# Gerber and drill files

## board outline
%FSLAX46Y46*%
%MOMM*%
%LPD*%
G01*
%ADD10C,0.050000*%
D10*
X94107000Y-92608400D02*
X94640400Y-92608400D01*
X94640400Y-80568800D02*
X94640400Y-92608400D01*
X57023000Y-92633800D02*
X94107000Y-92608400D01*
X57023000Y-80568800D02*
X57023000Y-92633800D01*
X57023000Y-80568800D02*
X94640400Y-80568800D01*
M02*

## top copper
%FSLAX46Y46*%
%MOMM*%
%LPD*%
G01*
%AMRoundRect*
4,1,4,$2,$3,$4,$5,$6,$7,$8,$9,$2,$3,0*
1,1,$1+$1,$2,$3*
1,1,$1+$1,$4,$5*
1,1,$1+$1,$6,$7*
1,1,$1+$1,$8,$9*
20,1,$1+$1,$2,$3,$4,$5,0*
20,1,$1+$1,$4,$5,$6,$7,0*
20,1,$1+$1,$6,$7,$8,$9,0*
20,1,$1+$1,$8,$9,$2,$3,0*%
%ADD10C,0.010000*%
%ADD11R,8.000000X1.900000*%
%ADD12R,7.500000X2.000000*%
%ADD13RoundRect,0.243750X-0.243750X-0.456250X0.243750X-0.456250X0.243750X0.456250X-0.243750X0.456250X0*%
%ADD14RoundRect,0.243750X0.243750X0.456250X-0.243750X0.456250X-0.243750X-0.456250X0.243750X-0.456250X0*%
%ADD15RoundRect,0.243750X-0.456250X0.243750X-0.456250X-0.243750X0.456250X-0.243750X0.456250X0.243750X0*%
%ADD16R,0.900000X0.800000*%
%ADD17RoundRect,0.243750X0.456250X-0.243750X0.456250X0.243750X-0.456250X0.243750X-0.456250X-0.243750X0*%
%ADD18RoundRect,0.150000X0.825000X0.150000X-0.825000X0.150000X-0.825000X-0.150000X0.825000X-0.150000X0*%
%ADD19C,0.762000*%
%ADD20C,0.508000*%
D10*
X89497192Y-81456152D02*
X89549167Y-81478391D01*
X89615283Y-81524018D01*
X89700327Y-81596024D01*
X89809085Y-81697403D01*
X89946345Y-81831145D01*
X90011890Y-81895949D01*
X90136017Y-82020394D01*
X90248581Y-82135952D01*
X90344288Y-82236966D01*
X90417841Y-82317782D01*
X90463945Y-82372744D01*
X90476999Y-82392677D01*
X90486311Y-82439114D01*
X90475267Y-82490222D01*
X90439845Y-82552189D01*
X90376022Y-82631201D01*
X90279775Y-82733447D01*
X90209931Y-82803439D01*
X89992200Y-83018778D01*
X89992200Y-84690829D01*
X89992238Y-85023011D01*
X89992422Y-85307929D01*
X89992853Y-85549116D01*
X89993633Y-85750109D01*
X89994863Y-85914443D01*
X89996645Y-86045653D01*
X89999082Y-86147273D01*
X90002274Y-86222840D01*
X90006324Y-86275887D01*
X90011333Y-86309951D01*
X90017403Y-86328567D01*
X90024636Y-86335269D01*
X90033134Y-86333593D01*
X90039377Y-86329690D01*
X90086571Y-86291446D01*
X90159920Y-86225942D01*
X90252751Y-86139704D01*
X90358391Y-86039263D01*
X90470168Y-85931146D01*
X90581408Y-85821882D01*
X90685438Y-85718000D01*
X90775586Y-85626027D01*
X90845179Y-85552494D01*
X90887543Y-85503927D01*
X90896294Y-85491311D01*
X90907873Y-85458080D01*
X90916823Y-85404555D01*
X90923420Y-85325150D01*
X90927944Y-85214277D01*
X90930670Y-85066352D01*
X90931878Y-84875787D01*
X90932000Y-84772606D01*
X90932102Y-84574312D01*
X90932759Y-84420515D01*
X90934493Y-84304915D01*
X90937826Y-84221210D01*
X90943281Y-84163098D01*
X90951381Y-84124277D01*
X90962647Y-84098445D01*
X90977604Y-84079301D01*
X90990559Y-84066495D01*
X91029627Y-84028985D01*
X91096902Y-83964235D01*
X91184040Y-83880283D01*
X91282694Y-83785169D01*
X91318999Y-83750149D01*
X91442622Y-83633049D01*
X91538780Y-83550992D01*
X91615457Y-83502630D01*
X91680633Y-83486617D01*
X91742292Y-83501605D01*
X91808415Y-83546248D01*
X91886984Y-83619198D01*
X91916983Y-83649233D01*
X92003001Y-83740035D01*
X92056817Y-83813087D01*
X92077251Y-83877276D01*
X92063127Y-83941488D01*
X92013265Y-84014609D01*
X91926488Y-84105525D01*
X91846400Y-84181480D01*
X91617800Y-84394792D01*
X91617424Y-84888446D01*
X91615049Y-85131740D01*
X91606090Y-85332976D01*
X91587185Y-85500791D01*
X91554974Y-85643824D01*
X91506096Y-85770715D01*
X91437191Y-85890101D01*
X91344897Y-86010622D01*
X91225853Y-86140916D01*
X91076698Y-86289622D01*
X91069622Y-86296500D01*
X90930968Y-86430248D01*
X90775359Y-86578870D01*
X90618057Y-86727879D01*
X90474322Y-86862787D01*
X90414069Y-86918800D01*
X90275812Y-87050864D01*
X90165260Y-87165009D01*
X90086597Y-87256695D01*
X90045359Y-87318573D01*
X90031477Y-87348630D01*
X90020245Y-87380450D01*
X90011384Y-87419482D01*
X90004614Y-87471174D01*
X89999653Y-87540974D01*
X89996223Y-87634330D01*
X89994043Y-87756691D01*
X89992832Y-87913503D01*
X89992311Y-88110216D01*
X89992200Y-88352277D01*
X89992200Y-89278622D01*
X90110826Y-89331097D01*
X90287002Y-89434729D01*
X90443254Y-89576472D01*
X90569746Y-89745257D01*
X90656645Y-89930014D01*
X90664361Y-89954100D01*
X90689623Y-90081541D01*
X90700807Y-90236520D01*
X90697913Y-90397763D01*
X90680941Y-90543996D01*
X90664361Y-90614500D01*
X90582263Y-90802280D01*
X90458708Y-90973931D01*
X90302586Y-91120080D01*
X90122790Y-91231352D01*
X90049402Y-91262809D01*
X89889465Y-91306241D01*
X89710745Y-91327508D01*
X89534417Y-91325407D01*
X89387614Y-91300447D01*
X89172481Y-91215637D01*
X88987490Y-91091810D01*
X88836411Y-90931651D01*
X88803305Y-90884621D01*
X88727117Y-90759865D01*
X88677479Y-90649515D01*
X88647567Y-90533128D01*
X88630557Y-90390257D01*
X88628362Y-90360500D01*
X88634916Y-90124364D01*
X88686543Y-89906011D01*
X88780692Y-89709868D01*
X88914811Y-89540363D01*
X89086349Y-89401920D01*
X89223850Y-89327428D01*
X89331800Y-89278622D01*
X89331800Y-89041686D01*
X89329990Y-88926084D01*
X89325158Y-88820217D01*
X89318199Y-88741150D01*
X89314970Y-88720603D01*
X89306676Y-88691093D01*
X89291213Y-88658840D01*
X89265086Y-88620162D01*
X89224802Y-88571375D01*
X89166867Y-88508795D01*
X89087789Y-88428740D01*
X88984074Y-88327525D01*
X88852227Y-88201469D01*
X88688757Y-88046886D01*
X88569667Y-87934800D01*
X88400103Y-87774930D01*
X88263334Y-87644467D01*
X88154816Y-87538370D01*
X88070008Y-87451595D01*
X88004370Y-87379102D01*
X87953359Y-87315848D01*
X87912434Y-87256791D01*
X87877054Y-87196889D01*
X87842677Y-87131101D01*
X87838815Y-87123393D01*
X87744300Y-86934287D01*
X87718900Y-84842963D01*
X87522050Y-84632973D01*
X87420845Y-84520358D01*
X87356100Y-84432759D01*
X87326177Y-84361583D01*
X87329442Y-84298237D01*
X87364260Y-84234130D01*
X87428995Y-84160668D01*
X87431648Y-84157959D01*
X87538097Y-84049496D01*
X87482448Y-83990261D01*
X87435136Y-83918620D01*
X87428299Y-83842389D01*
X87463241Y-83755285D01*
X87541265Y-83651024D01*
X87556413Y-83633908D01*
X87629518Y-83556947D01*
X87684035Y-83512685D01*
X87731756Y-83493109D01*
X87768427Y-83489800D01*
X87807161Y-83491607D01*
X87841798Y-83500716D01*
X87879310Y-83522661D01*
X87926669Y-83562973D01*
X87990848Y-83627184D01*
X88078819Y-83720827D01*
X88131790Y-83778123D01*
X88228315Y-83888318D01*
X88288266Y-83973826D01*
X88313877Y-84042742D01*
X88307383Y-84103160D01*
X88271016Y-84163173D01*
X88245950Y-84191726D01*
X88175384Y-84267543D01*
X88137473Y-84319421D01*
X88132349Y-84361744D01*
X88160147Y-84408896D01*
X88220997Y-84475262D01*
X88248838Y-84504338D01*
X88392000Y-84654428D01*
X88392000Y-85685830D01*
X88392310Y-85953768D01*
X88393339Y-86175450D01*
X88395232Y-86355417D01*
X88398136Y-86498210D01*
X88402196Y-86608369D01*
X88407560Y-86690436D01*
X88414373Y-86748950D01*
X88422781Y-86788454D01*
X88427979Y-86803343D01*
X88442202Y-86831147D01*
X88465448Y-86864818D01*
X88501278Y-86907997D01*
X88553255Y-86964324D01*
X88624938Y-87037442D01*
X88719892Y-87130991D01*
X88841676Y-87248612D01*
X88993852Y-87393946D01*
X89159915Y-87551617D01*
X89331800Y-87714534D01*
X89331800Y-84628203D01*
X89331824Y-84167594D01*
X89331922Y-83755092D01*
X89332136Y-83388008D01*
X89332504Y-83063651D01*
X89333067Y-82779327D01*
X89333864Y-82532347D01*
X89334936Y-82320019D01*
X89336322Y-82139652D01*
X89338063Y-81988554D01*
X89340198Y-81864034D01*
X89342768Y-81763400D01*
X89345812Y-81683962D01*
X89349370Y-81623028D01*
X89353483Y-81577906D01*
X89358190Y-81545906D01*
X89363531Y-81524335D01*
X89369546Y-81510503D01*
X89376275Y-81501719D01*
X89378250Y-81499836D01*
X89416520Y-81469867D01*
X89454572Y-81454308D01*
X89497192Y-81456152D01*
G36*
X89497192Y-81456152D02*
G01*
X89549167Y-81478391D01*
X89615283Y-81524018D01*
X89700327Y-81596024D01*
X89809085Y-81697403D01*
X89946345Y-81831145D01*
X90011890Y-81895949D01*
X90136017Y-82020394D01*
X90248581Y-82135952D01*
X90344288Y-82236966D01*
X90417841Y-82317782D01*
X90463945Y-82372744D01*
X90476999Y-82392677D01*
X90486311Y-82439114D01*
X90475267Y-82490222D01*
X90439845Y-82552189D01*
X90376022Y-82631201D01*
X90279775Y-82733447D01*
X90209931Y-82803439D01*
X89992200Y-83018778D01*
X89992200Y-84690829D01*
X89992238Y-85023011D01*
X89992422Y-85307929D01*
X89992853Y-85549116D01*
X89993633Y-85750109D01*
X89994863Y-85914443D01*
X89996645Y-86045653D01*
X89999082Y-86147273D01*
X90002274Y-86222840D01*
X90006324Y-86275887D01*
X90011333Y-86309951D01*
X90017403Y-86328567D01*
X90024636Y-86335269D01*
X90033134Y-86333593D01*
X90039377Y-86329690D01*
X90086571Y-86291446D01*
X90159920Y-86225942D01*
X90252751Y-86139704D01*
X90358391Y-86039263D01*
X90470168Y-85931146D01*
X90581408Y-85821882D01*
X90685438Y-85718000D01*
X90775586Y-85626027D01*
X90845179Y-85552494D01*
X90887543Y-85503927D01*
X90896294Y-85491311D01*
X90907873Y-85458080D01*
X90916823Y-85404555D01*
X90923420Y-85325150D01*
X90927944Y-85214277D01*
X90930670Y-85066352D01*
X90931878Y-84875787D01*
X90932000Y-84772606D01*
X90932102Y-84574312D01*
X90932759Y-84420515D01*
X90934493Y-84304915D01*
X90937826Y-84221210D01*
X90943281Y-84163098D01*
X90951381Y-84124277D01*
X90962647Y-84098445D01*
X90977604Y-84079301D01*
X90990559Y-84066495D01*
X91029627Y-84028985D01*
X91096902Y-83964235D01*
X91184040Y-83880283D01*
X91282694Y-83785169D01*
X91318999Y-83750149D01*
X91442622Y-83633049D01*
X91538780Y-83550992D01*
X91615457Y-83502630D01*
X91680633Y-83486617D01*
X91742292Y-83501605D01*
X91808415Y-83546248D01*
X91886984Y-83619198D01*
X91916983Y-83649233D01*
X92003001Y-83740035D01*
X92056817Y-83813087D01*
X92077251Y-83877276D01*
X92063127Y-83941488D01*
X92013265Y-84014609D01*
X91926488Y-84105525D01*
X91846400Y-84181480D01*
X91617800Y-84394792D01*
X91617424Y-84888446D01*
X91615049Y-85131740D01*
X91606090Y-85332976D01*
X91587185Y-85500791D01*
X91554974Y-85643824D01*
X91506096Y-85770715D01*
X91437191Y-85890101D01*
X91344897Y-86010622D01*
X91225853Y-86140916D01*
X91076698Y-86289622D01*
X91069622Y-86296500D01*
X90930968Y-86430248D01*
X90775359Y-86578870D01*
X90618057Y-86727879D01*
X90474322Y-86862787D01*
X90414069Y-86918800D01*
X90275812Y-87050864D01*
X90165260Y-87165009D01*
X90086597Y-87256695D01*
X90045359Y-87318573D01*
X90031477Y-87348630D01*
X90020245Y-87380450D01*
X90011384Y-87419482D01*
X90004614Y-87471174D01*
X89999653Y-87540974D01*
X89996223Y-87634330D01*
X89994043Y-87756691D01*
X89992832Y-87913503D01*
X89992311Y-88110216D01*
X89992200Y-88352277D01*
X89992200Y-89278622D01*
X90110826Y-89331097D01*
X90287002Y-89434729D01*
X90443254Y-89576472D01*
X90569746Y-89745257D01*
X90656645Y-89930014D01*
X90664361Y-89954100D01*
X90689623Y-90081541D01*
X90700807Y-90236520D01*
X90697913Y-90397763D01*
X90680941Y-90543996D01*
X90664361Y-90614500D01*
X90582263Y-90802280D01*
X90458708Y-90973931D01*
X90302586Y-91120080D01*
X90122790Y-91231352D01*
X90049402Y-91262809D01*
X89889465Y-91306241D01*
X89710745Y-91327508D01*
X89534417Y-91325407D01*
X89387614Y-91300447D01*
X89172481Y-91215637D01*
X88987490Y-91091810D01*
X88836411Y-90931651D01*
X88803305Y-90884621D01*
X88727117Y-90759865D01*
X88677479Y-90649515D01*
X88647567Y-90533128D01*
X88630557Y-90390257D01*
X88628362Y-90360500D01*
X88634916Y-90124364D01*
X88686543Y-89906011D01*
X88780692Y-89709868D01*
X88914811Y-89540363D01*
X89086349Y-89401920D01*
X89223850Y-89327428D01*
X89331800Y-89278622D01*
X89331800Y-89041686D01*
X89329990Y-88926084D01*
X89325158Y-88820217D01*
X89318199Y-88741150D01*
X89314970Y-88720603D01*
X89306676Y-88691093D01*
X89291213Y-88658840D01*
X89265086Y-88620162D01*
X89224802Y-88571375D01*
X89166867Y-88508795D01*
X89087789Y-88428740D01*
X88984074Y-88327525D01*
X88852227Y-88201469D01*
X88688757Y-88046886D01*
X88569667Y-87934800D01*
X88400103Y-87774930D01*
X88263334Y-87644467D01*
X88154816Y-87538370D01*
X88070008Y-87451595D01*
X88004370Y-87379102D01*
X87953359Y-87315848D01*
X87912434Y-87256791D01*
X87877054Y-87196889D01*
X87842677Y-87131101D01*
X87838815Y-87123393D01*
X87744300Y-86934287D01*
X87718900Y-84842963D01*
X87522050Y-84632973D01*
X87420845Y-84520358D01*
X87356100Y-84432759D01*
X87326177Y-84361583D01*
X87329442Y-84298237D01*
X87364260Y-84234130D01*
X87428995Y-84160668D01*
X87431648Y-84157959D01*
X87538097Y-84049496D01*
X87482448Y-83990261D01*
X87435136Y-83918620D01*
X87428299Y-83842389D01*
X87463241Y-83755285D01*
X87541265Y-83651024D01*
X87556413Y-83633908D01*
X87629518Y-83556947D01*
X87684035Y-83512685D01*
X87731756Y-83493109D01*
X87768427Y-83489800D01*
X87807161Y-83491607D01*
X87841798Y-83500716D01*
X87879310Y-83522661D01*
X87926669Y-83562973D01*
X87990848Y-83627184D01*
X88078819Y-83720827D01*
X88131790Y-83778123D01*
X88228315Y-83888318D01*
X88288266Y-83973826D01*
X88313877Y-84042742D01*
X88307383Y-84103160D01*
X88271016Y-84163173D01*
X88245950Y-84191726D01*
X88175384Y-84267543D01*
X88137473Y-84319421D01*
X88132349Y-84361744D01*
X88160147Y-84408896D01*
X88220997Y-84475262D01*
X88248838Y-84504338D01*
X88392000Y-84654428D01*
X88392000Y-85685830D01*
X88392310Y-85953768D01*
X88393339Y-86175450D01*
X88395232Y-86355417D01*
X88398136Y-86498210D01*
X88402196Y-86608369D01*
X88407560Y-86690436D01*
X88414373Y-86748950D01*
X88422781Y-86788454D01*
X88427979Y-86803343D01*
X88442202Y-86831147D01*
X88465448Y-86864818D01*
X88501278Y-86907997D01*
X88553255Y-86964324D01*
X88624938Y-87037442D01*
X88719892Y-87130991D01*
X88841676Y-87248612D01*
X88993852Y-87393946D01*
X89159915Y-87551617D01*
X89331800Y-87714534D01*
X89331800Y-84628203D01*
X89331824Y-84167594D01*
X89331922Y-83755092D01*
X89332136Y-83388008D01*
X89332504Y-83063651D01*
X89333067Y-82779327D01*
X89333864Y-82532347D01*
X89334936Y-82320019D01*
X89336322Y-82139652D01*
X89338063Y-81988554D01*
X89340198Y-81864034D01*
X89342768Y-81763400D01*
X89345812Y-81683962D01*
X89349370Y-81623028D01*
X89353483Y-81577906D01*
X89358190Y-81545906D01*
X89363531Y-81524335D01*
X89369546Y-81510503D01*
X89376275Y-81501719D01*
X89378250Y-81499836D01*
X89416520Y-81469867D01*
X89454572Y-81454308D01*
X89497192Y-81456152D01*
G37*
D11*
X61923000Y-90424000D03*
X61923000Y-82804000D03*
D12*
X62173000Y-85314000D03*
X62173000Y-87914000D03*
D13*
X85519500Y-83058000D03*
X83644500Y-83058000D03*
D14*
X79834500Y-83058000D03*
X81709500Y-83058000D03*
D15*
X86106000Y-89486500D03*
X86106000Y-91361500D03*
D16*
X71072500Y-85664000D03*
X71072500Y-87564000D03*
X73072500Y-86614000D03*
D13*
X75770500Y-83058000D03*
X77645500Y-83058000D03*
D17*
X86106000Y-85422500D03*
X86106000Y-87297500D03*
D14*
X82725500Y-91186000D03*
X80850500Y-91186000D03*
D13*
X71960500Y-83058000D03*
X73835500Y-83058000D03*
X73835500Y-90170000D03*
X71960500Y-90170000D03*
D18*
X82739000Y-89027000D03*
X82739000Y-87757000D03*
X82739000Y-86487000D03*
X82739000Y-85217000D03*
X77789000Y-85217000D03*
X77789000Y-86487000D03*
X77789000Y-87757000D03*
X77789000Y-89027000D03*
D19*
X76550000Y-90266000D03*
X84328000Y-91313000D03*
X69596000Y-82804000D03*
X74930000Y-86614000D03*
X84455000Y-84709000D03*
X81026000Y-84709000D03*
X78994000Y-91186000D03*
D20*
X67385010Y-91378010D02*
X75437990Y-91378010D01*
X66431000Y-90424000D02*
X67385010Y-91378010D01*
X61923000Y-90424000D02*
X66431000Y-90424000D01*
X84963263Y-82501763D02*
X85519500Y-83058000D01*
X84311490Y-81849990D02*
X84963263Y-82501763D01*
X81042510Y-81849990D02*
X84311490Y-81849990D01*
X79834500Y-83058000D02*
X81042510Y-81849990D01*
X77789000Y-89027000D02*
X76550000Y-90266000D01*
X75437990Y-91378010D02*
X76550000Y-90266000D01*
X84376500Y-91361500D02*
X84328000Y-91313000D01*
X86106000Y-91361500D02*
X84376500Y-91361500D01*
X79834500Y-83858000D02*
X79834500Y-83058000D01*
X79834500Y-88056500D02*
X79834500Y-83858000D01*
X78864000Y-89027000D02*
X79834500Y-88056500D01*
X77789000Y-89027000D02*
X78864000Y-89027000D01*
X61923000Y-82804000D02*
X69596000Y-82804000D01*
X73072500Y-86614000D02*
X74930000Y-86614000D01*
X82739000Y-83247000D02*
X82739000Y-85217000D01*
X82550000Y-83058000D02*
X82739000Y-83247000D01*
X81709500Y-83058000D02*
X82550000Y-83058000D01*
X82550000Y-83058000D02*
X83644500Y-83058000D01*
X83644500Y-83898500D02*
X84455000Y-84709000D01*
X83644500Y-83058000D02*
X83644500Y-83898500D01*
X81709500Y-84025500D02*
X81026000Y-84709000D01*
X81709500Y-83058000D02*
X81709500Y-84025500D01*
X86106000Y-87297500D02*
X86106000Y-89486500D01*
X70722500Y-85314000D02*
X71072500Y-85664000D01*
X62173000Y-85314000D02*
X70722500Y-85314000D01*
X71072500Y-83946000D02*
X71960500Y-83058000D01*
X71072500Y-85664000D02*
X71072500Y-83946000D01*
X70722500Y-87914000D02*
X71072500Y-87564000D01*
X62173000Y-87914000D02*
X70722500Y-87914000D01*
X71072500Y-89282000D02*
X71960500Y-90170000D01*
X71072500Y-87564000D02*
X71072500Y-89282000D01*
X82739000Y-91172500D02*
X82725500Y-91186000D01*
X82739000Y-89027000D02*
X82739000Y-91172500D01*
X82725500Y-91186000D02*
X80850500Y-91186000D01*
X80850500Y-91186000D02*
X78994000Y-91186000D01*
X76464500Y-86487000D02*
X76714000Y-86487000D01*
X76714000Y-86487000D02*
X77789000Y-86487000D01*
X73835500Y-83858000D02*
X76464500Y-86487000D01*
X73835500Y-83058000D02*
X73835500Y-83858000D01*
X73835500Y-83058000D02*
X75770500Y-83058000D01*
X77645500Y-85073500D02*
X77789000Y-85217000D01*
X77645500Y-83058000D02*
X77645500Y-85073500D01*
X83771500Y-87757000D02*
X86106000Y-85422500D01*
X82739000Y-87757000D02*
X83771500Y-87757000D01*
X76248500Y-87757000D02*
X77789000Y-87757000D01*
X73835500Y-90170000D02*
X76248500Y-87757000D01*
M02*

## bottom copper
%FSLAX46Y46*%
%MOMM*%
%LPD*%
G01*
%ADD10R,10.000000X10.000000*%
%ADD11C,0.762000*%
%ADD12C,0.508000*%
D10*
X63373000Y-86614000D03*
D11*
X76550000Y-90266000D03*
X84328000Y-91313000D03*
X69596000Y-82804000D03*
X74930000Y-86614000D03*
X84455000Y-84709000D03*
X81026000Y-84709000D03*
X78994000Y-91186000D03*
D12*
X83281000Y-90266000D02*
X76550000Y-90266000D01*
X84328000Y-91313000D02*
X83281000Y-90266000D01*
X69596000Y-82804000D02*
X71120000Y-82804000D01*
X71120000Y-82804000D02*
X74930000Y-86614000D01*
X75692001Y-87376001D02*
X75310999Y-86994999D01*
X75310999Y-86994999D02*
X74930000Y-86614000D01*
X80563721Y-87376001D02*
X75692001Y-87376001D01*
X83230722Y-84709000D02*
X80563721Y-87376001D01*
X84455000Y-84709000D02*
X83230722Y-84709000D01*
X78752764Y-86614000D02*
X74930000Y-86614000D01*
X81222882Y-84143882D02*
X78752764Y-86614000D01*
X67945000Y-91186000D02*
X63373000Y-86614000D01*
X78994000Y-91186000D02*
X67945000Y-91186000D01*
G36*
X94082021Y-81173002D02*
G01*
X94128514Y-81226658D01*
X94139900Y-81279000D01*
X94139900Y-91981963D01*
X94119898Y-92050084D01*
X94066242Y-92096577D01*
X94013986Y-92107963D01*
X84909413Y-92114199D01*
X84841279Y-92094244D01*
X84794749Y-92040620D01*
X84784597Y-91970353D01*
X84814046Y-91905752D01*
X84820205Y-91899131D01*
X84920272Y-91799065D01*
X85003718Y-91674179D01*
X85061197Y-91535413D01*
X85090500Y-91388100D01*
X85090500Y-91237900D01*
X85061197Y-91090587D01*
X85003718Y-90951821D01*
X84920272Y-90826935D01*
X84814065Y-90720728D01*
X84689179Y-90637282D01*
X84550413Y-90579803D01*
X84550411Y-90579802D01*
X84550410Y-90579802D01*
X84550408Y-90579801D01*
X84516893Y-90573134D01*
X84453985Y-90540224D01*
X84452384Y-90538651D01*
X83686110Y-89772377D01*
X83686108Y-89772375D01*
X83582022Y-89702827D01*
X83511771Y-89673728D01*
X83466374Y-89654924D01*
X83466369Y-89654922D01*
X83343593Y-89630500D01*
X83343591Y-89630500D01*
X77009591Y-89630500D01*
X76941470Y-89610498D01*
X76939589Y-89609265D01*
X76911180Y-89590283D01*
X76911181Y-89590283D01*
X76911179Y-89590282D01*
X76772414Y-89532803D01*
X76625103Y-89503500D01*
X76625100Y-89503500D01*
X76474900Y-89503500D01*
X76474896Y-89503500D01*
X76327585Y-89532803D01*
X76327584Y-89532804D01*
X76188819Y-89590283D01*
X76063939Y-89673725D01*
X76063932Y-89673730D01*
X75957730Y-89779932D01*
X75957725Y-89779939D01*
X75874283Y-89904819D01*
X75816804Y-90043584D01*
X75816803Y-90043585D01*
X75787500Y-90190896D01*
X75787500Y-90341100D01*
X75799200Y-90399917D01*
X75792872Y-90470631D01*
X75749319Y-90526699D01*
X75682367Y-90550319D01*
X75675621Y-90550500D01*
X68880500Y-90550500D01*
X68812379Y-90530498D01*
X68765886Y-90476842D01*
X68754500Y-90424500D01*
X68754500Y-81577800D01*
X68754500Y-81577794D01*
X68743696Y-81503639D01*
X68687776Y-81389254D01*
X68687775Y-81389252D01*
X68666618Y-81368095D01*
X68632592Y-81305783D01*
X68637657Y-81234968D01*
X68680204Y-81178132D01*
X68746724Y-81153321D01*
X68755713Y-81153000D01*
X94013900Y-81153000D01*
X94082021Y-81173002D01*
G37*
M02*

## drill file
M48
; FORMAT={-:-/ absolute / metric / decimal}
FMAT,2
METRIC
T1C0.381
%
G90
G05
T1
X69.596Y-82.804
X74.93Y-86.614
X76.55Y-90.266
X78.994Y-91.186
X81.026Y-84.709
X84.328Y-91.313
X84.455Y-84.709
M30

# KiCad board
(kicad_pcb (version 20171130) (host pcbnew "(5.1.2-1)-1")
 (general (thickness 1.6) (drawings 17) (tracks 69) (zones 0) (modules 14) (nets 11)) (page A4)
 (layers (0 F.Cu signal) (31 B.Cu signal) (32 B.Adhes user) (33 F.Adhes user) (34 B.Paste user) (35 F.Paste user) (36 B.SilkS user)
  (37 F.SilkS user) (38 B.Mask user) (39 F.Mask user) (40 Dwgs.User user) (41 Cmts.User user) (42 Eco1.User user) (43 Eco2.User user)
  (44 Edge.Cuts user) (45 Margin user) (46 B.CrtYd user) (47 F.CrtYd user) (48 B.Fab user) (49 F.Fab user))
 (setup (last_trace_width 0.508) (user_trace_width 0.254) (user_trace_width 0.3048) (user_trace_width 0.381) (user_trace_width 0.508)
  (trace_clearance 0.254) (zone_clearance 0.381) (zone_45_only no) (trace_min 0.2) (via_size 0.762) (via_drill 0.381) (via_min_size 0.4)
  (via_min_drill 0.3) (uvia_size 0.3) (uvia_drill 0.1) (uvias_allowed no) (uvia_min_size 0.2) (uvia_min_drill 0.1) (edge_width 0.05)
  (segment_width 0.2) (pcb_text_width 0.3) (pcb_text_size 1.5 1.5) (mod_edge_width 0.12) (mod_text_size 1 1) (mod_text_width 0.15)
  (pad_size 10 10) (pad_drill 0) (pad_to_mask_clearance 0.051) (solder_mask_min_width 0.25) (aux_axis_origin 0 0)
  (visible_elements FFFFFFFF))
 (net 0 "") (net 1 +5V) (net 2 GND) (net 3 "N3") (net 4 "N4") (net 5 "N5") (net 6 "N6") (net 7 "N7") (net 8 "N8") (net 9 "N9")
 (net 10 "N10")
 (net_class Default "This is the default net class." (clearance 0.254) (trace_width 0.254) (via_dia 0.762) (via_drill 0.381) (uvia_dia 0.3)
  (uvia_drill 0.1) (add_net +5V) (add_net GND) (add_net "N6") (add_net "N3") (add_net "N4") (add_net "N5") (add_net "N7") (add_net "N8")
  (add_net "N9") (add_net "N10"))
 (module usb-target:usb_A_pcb (layer F.Cu) (at 57.023 86.614 270)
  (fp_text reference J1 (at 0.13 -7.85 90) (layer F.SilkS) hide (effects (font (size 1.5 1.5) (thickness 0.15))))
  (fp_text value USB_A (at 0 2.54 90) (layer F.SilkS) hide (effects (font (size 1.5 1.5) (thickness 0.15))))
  (pad 1 connect rect (at 3.81 -4.9 270) (size 1.9 8) (layers F.Cu F.Mask) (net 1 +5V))
  (pad 4 connect rect (at -3.81 -4.9 270) (size 1.9 8) (layers F.Cu F.Mask) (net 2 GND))
  (pad 3 connect rect (at -1.3 -5.15 270) (size 2 7.5) (layers F.Cu F.Mask) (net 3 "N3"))
  (pad 2 connect rect (at 1.3 -5.15 270) (size 2 7.5) (layers F.Cu F.Mask) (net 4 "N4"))
  (pad 5 smd rect (at 0 -6.35 270) (size 10 10) (layers B.Cu B.Mask) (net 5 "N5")))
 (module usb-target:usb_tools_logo (layer F.Cu) (at 89.662 86.36)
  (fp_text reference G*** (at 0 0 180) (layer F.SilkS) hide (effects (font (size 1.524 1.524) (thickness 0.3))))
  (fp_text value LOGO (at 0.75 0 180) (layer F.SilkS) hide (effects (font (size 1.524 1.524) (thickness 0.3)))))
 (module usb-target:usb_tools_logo (layer F.Cu) (at 89.662 86.36)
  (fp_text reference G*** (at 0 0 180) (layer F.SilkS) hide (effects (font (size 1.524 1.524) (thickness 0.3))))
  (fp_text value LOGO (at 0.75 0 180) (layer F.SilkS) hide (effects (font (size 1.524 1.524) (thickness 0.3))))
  (fp_poly
   (pts (xy -0.164808 -4.903848) (xy -0.112833 -4.881609) (xy -0.046717 -4.835982) (xy 0.038327 -4.763976) (xy 0.147085 -4.662597)
    (xy 0.284345 -4.528855) (xy 0.34989 -4.464051) (xy 0.474017 -4.339606) (xy 0.586581 -4.224048) (xy 0.682288 -4.123034)
    (xy 0.755841 -4.042218) (xy 0.801945 -3.987256) (xy 0.814999 -3.967323) (xy 0.824311 -3.920886) (xy 0.813267 -3.869778)
    (xy 0.777845 -3.807811) (xy 0.714022 -3.728799) (xy 0.617775 -3.626553) (xy 0.547931 -3.556561) (xy 0.3302 -3.341222)
    (xy 0.3302 -1.669171) (xy 0.330238 -1.336989) (xy 0.330422 -1.052071) (xy 0.330853 -0.810884) (xy 0.331633 -0.609891)
    (xy 0.332863 -0.445557) (xy 0.334645 -0.314347) (xy 0.337082 -0.212727) (xy 0.340274 -0.13716) (xy 0.344324 -0.084113)
    (xy 0.349333 -0.050049) (xy 0.355403 -0.031433) (xy 0.362636 -0.024731) (xy 0.371134 -0.026407) (xy 0.377377 -0.03031)
    (xy 0.424571 -0.068554) (xy 0.49792 -0.134058) (xy 0.590751 -0.220296) (xy 0.696391 -0.320737) (xy 0.808168 -0.428854)
    (xy 0.919408 -0.538118) (xy 1.023438 -0.642) (xy 1.113586 -0.733973) (xy 1.183179 -0.807506) (xy 1.225543 -0.856073)
    (xy 1.234294 -0.868689) (xy 1.245873 -0.90192) (xy 1.254823 -0.955445) (xy 1.26142 -1.03485) (xy 1.265944 -1.145723)
    (xy 1.26867 -1.293648) (xy 1.269878 -1.484213) (xy 1.27 -1.587394) (xy 1.270102 -1.785688) (xy 1.270759 -1.939485)
    (xy 1.272493 -2.055085) (xy 1.275826 -2.13879) (xy 1.281281 -2.196902) (xy 1.289381 -2.235723) (xy 1.300647 -2.261555)
    (xy 1.315604 -2.280699) (xy 1.328559 -2.293505) (xy 1.367627 -2.331015) (xy 1.434902 -2.395765) (xy 1.52204 -2.479717)
    (xy 1.620694 -2.574831) (xy 1.656999 -2.609851) (xy 1.780622 -2.726951) (xy 1.87678 -2.809008) (xy 1.953457 -2.85737)
    (xy 2.018633 -2.873383) (xy 2.080292 -2.858395) (xy 2.146415 -2.813752) (xy 2.224984 -2.740802) (xy 2.254983 -2.710767)
    (xy 2.341001 -2.619965) (xy 2.394817 -2.546913) (xy 2.415251 -2.482724) (xy 2.401127 -2.418512) (xy 2.351265 -2.345391)
    (xy 2.264488 -2.254475) (xy 2.1844 -2.17852) (xy 1.9558 -1.965208) (xy 1.955424 -1.471554) (xy 1.953049 -1.22826) (xy 1.94409 -1.027024)
    (xy 1.925185 -0.859209) (xy 1.892974 -0.716176) (xy 1.844096 -0.589285) (xy 1.775191 -0.469899) (xy 1.682897 -0.349378)
    (xy 1.563853 -0.219084) (xy 1.414698 -0.070378) (xy 1.407622 -0.0635) (xy 1.268968 0.070248) (xy 1.113359 0.21887)
    (xy 0.956057 0.367879) (xy 0.812322 0.502787) (xy 0.752069 0.5588) (xy 0.613812 0.690864) (xy 0.50326 0.805009) (xy 0.424597 0.896695)
    (xy 0.383359 0.958573) (xy 0.369477 0.98863) (xy 0.358245 1.02045) (xy 0.349384 1.059482) (xy 0.342614 1.111174) (xy 0.337653 1.180974)
    (xy 0.334223 1.27433) (xy 0.332043 1.396691) (xy 0.330832 1.553503) (xy 0.330311 1.750216) (xy 0.3302 1.992277) (xy 0.3302 2.918622)
    (xy 0.448826 2.971097) (xy 0.625002 3.074729) (xy 0.781254 3.216472) (xy 0.907746 3.385257) (xy 0.994645 3.570014) (xy 1.002361 3.5941)
    (xy 1.027623 3.721541) (xy 1.038807 3.87652) (xy 1.035913 4.037763) (xy 1.018941 4.183996) (xy 1.002361 4.2545) (xy 0.920263 4.44228)
    (xy 0.796708 4.613931) (xy 0.640586 4.76008) (xy 0.46079 4.871352) (xy 0.387402 4.902809) (xy 0.227465 4.946241) (xy 0.048745 4.967508)
    (xy -0.127583 4.965407) (xy -0.274386 4.940447) (xy -0.489519 4.855637) (xy -0.67451 4.73181) (xy -0.825589 4.571651)
    (xy -0.858695 4.524621) (xy -0.934883 4.399865) (xy -0.984521 4.289515) (xy -1.014433 4.173128) (xy -1.031443 4.030257)
    (xy -1.033638 4.0005) (xy -1.027084 3.764364) (xy -0.975457 3.546011) (xy -0.881308 3.349868) (xy -0.747189 3.180363)
    (xy -0.575651 3.04192) (xy -0.43815 2.967428) (xy -0.3302 2.918622) (xy -0.3302 2.681686) (xy -0.33201 2.566084) (xy -0.336842 2.460217)
    (xy -0.343801 2.38115) (xy -0.34703 2.360603) (xy -0.355324 2.331093) (xy -0.370787 2.29884) (xy -0.396914 2.260162)
    (xy -0.437198 2.211375) (xy -0.495133 2.148795) (xy -0.574211 2.06874) (xy -0.677926 1.967525) (xy -0.809773 1.841469)
    (xy -0.973243 1.686886) (xy -1.092333 1.5748) (xy -1.261897 1.41493) (xy -1.398666 1.284467) (xy -1.507184 1.17837)
    (xy -1.591992 1.091595) (xy -1.65763 1.019102) (xy -1.708641 0.955848) (xy -1.749566 0.896791) (xy -1.784946 0.836889)
    (xy -1.819323 0.771101) (xy -1.823185 0.763393) (xy -1.9177 0.574287) (xy -1.9431 -1.517037) (xy -2.13995 -1.727027)
    (xy -2.241155 -1.839642) (xy -2.3059 -1.927241) (xy -2.335823 -1.998417) (xy -2.332558 -2.061763) (xy -2.29774 -2.12587)
    (xy -2.233005 -2.199332) (xy -2.230352 -2.202041) (xy -2.123903 -2.310504) (xy -2.179552 -2.369739) (xy -2.226864 -2.44138)
    (xy -2.233701 -2.517611) (xy -2.198759 -2.604715) (xy -2.120735 -2.708976) (xy -2.105587 -2.726092) (xy -2.032482 -2.803053)
    (xy -1.977965 -2.847315) (xy -1.930244 -2.866891) (xy -1.893573 -2.8702) (xy -1.854839 -2.868393) (xy -1.820202 -2.859284)
    (xy -1.78269 -2.837339) (xy -1.735331 -2.797027) (xy -1.671152 -2.732816) (xy -1.583181 -2.639173) (xy -1.53021 -2.581877)
    (xy -1.433685 -2.471682) (xy -1.373734 -2.386174) (xy -1.348123 -2.317258) (xy -1.354617 -2.25684) (xy -1.390984 -2.196827)
    (xy -1.41605 -2.168274) (xy -1.486616 -2.092457) (xy -1.524527 -2.040579) (xy -1.529651 -1.998256) (xy -1.501853 -1.951104)
    (xy -1.441003 -1.884738) (xy -1.413162 -1.855662) (xy -1.27 -1.705572) (xy -1.27 -0.67417) (xy -1.26969 -0.406232)
    (xy -1.268661 -0.18455) (xy -1.266768 -0.004583) (xy -1.263864 0.13821) (xy -1.259804 0.248369) (xy -1.25444 0.330436)
    (xy -1.247627 0.38895) (xy -1.239219 0.428454) (xy -1.234021 0.443343) (xy -1.219798 0.471147) (xy -1.196552 0.504818)
    (xy -1.160722 0.547997) (xy -1.108745 0.604324) (xy -1.037062 0.677442) (xy -0.942108 0.770991) (xy -0.820324 0.888612)
    (xy -0.668148 1.033946) (xy -0.502085 1.191617) (xy -0.3302 1.354534) (xy -0.3302 -1.731797) (xy -0.330176 -2.192406)
    (xy -0.330078 -2.604908) (xy -0.329864 -2.971992) (xy -0.329496 -3.296349) (xy -0.328933 -3.580673) (xy -0.328136 -3.827653)
    (xy -0.327064 -4.039981) (xy -0.325678 -4.220348) (xy -0.323937 -4.371446) (xy -0.321802 -4.495966) (xy -0.319232 -4.5966)
    (xy -0.316188 -4.676038) (xy -0.31263 -4.736972) (xy -0.308517 -4.782094) (xy -0.30381 -4.814094) (xy -0.298469 -4.835665)
    (xy -0.292454 -4.849497) (xy -0.285725 -4.858281) (xy -0.28375 -4.860164) (xy -0.24548 -4.890133) (xy -0.207428 -4.905692)
    (xy -0.164808 -4.903848))
   (layer F.Cu) (width 0.01)))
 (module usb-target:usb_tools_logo (layer B.Cu) (at 91.567 86.487 180)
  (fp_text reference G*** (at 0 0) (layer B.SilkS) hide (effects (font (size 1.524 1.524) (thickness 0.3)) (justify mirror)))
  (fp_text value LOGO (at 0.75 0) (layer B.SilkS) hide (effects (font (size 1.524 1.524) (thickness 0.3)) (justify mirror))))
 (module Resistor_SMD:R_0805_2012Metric (layer F.Cu) (at 84.582 83.058)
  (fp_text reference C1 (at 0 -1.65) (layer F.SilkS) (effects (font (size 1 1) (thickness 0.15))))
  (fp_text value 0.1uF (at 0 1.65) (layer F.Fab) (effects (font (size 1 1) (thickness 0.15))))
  (pad 2 smd roundrect (at 0.9375 0) (size 0.975 1.4) (layers F.Cu F.Paste F.Mask) (roundrect_rratio 0.25) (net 1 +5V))
  (pad 1 smd roundrect (at -0.9375 0) (size 0.975 1.4) (layers F.Cu F.Paste F.Mask) (roundrect_rratio 0.25) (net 2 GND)))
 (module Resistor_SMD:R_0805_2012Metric (layer F.Cu) (at 80.772 83.058 180)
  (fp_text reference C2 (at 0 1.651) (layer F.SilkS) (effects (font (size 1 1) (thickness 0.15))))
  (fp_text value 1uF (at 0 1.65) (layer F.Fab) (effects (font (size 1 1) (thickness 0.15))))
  (pad 2 smd roundrect (at 0.9375 0 180) (size 0.975 1.4) (layers F.Cu F.Paste F.Mask) (roundrect_rratio 0.25) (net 1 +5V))
  (pad 1 smd roundrect (at -0.9375 0 180) (size 0.975 1.4) (layers F.Cu F.Paste F.Mask) (roundrect_rratio 0.25) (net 2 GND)))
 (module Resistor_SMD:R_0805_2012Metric (layer F.Cu) (at 86.106 90.424 270)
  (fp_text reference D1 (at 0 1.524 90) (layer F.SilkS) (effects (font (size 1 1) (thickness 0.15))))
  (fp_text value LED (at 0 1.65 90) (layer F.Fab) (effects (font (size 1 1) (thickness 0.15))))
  (pad 1 smd roundrect (at -0.9375 0 270) (size 0.975 1.4) (layers F.Cu F.Paste F.Mask) (roundrect_rratio 0.25) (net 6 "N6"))
  (pad 2 smd roundrect (at 0.9375 0 270) (size 0.975 1.4) (layers F.Cu F.Paste F.Mask) (roundrect_rratio 0.25) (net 1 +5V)))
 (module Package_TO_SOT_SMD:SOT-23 (layer F.Cu) (at 72.0725 86.614)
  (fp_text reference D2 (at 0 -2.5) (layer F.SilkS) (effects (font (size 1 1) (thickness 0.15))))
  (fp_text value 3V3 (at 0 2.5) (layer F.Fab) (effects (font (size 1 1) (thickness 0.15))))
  (pad 1 smd rect (at -1 -0.95) (size 0.9 0.8) (layers F.Cu F.Paste F.Mask) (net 3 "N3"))
  (pad 2 smd rect (at -1 0.95) (size 0.9 0.8) (layers F.Cu F.Paste F.Mask) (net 4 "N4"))
  (pad 3 smd rect (at 1 0) (size 0.9 0.8) (layers F.Cu F.Paste F.Mask) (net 2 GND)))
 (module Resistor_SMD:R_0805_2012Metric (layer F.Cu) (at 76.708 83.058)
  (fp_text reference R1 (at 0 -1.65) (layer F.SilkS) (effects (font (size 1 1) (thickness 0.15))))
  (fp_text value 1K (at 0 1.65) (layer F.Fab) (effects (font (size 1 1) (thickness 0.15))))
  (pad 1 smd roundrect (at -0.9375 0) (size 0.975 1.4) (layers F.Cu F.Paste F.Mask) (roundrect_rratio 0.25) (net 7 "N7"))
  (pad 2 smd roundrect (at 0.9375 0) (size 0.975 1.4) (layers F.Cu F.Paste F.Mask) (roundrect_rratio 0.25) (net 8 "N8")))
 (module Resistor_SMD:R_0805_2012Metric (layer F.Cu) (at 86.106 86.36 90)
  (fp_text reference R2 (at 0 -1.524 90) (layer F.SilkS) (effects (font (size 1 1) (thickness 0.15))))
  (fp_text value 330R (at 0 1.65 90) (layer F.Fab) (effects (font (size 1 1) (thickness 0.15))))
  (pad 2 smd roundrect (at 0.9375 0 90) (size 0.975 1.4) (layers F.Cu F.Paste F.Mask) (roundrect_rratio 0.25) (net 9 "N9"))
  (pad 1 smd roundrect (at -0.9375 0 90) (size 0.975 1.4) (layers F.Cu F.Paste F.Mask) (roundrect_rratio 0.25) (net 6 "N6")))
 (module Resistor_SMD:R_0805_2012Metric (layer F.Cu) (at 81.788 91.186 180)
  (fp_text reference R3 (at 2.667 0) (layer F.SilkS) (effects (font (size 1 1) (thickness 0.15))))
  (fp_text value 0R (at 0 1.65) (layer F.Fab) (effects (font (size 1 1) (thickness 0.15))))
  (pad 1 smd roundrect (at -0.9375 0 180) (size 0.975 1.4) (layers F.Cu F.Paste F.Mask) (roundrect_rratio 0.25) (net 5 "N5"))
  (pad 2 smd roundrect (at 0.9375 0 180) (size 0.975 1.4) (layers F.Cu F.Paste F.Mask) (roundrect_rratio 0.25) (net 5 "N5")))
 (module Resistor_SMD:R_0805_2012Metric (layer F.Cu) (at 72.898 83.058)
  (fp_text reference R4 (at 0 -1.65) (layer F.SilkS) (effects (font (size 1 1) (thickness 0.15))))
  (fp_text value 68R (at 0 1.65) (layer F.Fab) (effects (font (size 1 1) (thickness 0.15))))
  (pad 1 smd roundrect (at -0.9375 0) (size 0.975 1.4) (layers F.Cu F.Paste F.Mask) (roundrect_rratio 0.25) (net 3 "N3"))
  (pad 2 smd roundrect (at 0.9375 0) (size 0.975 1.4) (layers F.Cu F.Paste F.Mask) (roundrect_rratio 0.25) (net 7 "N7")))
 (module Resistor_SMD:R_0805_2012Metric (layer F.Cu) (at 72.898 90.17)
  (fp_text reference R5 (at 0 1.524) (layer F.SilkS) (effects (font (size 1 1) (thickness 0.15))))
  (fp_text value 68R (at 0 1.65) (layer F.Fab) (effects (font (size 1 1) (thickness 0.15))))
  (pad 2 smd roundrect (at 0.9375 0) (size 0.975 1.4) (layers F.Cu F.Paste F.Mask) (roundrect_rratio 0.25) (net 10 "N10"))
  (pad 1 smd roundrect (at -0.9375 0) (size 0.975 1.4) (layers F.Cu F.Paste F.Mask) (roundrect_rratio 0.25) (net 4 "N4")))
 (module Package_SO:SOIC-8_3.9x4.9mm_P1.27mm (layer F.Cu) (at 80.264 87.122 180)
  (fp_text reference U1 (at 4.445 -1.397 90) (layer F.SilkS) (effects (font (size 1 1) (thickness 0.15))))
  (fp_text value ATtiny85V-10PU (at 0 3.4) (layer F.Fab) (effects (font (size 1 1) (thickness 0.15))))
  (pad 1 smd roundrect (at -2.475 -1.905 180) (size 1.95 0.6) (layers F.Cu F.Paste F.Mask) (roundrect_rratio 0.25) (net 5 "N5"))
  (pad 2 smd roundrect (at -2.475 -0.635 180) (size 1.95 0.6) (layers F.Cu F.Paste F.Mask) (roundrect_rratio 0.25) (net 9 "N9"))
  (pad 3 smd roundrect (at -2.475 0.635 180) (size 1.95 0.6) (layers F.Cu F.Paste F.Mask) (roundrect_rratio 0.25))
  (pad 4 smd roundrect (at -2.475 1.905 180) (size 1.95 0.6) (layers F.Cu F.Paste F.Mask) (roundrect_rratio 0.25) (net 2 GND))
  (pad 5 smd roundrect (at 2.475 1.905 180) (size 1.95 0.6) (layers F.Cu F.Paste F.Mask) (roundrect_rratio 0.25) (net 8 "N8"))
  (pad 6 smd roundrect (at 2.475 0.635 180) (size 1.95 0.6) (layers F.Cu F.Paste F.Mask) (roundrect_rratio 0.25) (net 7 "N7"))
  (pad 7 smd roundrect (at 2.475 -0.635 180) (size 1.95 0.6) (layers F.Cu F.Paste F.Mask) (roundrect_rratio 0.25) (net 10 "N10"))
  (pad 8 smd roundrect (at 2.475 -1.905 180) (size 1.95 0.6) (layers F.Cu F.Paste F.Mask) (roundrect_rratio 0.25) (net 1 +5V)))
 (gr_line (start 94.107 92.6084) (end 94.6404 92.6084) (layer Edge.Cuts) (width 0.05))
 (gr_line (start 94.6404 80.5688) (end 94.6404 92.6084) (layer Edge.Cuts) (width 0.05))
 (gr_line (start 57.023 92.6338) (end 94.107 92.6084) (layer Edge.Cuts) (width 0.05))
 (gr_line (start 57.023 80.5688) (end 57.023 92.6338) (layer Edge.Cuts) (width 0.05))
 (gr_line (start 57.023 80.5688) (end 94.6404 80.5688) (layer Edge.Cuts) (width 0.05))
 (segment (start 67.38501 91.37801) (end 75.43799 91.37801) (width 0.508) (layer F.Cu) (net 1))
 (segment (start 66.431 90.424) (end 67.38501 91.37801) (width 0.508) (layer F.Cu) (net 1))
 (segment (start 61.923 90.424) (end 66.431 90.424) (width 0.508) (layer F.Cu) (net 1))
 (segment (start 84.963263 82.501763) (end 85.5195 83.058) (width 0.508) (layer F.Cu) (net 1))
 (segment (start 84.31149 81.84999) (end 84.963263 82.501763) (width 0.508) (layer F.Cu) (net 1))
 (segment (start 81.04251 81.84999) (end 84.31149 81.84999) (width 0.508) (layer F.Cu) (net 1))
 (segment (start 79.8345 83.058) (end 81.04251 81.84999) (width 0.508) (layer F.Cu) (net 1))
 (via (at 76.55 90.266) (size 0.762) (drill 0.381) (layers F.Cu B.Cu) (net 1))
 (segment (start 77.789 89.027) (end 76.55 90.266) (width 0.508) (layer F.Cu) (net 1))
 (segment (start 75.43799 91.37801) (end 76.55 90.266) (width 0.508) (layer F.Cu) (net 1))
 (via (at 84.328 91.313) (size 0.762) (drill 0.381) (layers F.Cu B.Cu) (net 1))
 (segment (start 84.3765 91.3615) (end 84.328 91.313) (width 0.508) (layer F.Cu) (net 1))
 (segment (start 86.106 91.3615) (end 84.3765 91.3615) (width 0.508) (layer F.Cu) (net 1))
 (segment (start 83.281 90.266) (end 76.55 90.266) (width 0.508) (layer B.Cu) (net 1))
 (segment (start 84.328 91.313) (end 83.281 90.266) (width 0.508) (layer B.Cu) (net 1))
 (segment (start 79.8345 83.858) (end 79.8345 83.058) (width 0.508) (layer F.Cu) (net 1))
 (segment (start 79.8345 88.0565) (end 79.8345 83.858) (width 0.508) (layer F.Cu) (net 1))
 (segment (start 78.864 89.027) (end 79.8345 88.0565) (width 0.508) (layer F.Cu) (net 1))
 (segment (start 77.789 89.027) (end 78.864 89.027) (width 0.508) (layer F.Cu) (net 1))
 (via (at 69.596 82.804) (size 0.762) (drill 0.381) (layers F.Cu B.Cu) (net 2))
 (segment (start 61.923 82.804) (end 69.596 82.804) (width 0.508) (layer F.Cu) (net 2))
 (segment (start 69.596 82.804) (end 71.12 82.804) (width 0.508) (layer B.Cu) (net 2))
 (segment (start 71.12 82.804) (end 74.93 86.614) (width 0.508) (layer B.Cu) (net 2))
 (via (at 74.93 86.614) (size 0.762) (drill 0.381) (layers F.Cu B.Cu) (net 2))
 (segment (start 73.0725 86.614) (end 74.93 86.614) (width 0.508) (layer F.Cu) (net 2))
 (segment (start 82.739 83.247) (end 82.739 85.217) (width 0.508) (layer F.Cu) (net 2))
 (segment (start 82.55 83.058) (end 82.739 83.247) (width 0.508) (layer F.Cu) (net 2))
 (segment (start 81.7095 83.058) (end 82.55 83.058) (width 0.508) (layer F.Cu) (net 2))
 (segment (start 82.55 83.058) (end 83.6445 83.058) (width 0.508) (layer F.Cu) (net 2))
 (via (at 84.455 84.709) (size 0.762) (drill 0.381) (layers F.Cu B.Cu) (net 2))
 (segment (start 83.6445 83.8985) (end 84.455 84.709) (width 0.508) (layer F.Cu) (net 2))
 (segment (start 83.6445 83.058) (end 83.6445 83.8985) (width 0.508) (layer F.Cu) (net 2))
 (segment (start 75.692001 87.376001) (end 75.310999 86.994999) (width 0.508) (layer B.Cu) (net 2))
 (segment (start 75.310999 86.994999) (end 74.93 86.614) (width 0.508) (layer B.Cu) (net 2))
 (segment (start 80.563721 87.376001) (end 75.692001 87.376001) (width 0.508) (layer B.Cu) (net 2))
 (segment (start 83.230722 84.709) (end 80.563721 87.376001) (width 0.508) (layer B.Cu) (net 2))
 (segment (start 84.455 84.709) (end 83.230722 84.709) (width 0.508) (layer B.Cu) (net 2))
 (segment (start 78.752764 86.614) (end 74.93 86.614) (width 0.508) (layer B.Cu) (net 2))
 (segment (start 81.222882 84.143882) (end 78.752764 86.614) (width 0.508) (layer B.Cu) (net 2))
 (segment (start 81.7095 84.0255) (end 81.026 84.709) (width 0.508) (layer F.Cu) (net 2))
 (via (at 81.026 84.709) (size 0.762) (drill 0.381) (layers F.Cu B.Cu) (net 2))
 (segment (start 81.7095 83.058) (end 81.7095 84.0255) (width 0.508) (layer F.Cu) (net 2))
 (segment (start 86.106 87.2975) (end 86.106 89.4865) (width 0.508) (layer F.Cu) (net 6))
 (segment (start 70.7225 85.314) (end 71.0725 85.664) (width 0.508) (layer F.Cu) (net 3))
 (segment (start 62.173 85.314) (end 70.7225 85.314) (width 0.508) (layer F.Cu) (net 3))
 (segment (start 71.0725 83.946) (end 71.9605 83.058) (width 0.508) (layer F.Cu) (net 3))
 (segment (start 71.0725 85.664) (end 71.0725 83.946) (width 0.508) (layer F.Cu) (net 3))
 (segment (start 70.7225 87.914) (end 71.0725 87.564) (width 0.508) (layer F.Cu) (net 4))
 (segment (start 62.173 87.914) (end 70.7225 87.914) (width 0.508) (layer F.Cu) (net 4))
 (segment (start 71.0725 89.282) (end 71.9605 90.17) (width 0.508) (layer F.Cu) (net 4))
 (segment (start 71.0725 87.564) (end 71.0725 89.282) (width 0.508) (layer F.Cu) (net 4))
 (segment (start 82.739 91.1725) (end 82.7255 91.186) (width 0.508) (layer F.Cu) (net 5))
 (segment (start 82.739 89.027) (end 82.739 91.1725) (width 0.508) (layer F.Cu) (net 5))
 (segment (start 82.7255 91.186) (end 80.8505 91.186) (width 0.508) (layer F.Cu) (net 5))
 (via (at 78.994 91.186) (size 0.762) (drill 0.381) (layers F.Cu B.Cu) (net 5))
 (segment (start 80.8505 91.186) (end 78.994 91.186) (width 0.508) (layer F.Cu) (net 5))
 (segment (start 67.945 91.186) (end 63.373 86.614) (width 0.508) (layer B.Cu) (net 5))
 (segment (start 78.994 91.186) (end 67.945 91.186) (width 0.508) (layer B.Cu) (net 5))
 (segment (start 76.4645 86.487) (end 76.714 86.487) (width 0.508) (layer F.Cu) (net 7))
 (segment (start 76.714 86.487) (end 77.789 86.487) (width 0.508) (layer F.Cu) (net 7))
 (segment (start 73.8355 83.858) (end 76.4645 86.487) (width 0.508) (layer F.Cu) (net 7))
 (segment (start 73.8355 83.058) (end 73.8355 83.858) (width 0.508) (layer F.Cu) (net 7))
 (segment (start 73.8355 83.058) (end 75.7705 83.058) (width 0.508) (layer F.Cu) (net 7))
 (segment (start 77.6455 85.0735) (end 77.789 85.217) (width 0.508) (layer F.Cu) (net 8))
 (segment (start 77.6455 83.058) (end 77.6455 85.0735) (width 0.508) (layer F.Cu) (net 8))
 (segment (start 83.7715 87.757) (end 86.106 85.4225) (width 0.508) (layer F.Cu) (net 9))
 (segment (start 82.739 87.757) (end 83.7715 87.757) (width 0.508) (layer F.Cu) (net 9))
 (segment (start 76.2485 87.757) (end 77.789 87.757) (width 0.508) (layer F.Cu) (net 10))
 (segment (start 73.8355 90.17) (end 76.2485 87.757) (width 0.508) (layer F.Cu) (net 10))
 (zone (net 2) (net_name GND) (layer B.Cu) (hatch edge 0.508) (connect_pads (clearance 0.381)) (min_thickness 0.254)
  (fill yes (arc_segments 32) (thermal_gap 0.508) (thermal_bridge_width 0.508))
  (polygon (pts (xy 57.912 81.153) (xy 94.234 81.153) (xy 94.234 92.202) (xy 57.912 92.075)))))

